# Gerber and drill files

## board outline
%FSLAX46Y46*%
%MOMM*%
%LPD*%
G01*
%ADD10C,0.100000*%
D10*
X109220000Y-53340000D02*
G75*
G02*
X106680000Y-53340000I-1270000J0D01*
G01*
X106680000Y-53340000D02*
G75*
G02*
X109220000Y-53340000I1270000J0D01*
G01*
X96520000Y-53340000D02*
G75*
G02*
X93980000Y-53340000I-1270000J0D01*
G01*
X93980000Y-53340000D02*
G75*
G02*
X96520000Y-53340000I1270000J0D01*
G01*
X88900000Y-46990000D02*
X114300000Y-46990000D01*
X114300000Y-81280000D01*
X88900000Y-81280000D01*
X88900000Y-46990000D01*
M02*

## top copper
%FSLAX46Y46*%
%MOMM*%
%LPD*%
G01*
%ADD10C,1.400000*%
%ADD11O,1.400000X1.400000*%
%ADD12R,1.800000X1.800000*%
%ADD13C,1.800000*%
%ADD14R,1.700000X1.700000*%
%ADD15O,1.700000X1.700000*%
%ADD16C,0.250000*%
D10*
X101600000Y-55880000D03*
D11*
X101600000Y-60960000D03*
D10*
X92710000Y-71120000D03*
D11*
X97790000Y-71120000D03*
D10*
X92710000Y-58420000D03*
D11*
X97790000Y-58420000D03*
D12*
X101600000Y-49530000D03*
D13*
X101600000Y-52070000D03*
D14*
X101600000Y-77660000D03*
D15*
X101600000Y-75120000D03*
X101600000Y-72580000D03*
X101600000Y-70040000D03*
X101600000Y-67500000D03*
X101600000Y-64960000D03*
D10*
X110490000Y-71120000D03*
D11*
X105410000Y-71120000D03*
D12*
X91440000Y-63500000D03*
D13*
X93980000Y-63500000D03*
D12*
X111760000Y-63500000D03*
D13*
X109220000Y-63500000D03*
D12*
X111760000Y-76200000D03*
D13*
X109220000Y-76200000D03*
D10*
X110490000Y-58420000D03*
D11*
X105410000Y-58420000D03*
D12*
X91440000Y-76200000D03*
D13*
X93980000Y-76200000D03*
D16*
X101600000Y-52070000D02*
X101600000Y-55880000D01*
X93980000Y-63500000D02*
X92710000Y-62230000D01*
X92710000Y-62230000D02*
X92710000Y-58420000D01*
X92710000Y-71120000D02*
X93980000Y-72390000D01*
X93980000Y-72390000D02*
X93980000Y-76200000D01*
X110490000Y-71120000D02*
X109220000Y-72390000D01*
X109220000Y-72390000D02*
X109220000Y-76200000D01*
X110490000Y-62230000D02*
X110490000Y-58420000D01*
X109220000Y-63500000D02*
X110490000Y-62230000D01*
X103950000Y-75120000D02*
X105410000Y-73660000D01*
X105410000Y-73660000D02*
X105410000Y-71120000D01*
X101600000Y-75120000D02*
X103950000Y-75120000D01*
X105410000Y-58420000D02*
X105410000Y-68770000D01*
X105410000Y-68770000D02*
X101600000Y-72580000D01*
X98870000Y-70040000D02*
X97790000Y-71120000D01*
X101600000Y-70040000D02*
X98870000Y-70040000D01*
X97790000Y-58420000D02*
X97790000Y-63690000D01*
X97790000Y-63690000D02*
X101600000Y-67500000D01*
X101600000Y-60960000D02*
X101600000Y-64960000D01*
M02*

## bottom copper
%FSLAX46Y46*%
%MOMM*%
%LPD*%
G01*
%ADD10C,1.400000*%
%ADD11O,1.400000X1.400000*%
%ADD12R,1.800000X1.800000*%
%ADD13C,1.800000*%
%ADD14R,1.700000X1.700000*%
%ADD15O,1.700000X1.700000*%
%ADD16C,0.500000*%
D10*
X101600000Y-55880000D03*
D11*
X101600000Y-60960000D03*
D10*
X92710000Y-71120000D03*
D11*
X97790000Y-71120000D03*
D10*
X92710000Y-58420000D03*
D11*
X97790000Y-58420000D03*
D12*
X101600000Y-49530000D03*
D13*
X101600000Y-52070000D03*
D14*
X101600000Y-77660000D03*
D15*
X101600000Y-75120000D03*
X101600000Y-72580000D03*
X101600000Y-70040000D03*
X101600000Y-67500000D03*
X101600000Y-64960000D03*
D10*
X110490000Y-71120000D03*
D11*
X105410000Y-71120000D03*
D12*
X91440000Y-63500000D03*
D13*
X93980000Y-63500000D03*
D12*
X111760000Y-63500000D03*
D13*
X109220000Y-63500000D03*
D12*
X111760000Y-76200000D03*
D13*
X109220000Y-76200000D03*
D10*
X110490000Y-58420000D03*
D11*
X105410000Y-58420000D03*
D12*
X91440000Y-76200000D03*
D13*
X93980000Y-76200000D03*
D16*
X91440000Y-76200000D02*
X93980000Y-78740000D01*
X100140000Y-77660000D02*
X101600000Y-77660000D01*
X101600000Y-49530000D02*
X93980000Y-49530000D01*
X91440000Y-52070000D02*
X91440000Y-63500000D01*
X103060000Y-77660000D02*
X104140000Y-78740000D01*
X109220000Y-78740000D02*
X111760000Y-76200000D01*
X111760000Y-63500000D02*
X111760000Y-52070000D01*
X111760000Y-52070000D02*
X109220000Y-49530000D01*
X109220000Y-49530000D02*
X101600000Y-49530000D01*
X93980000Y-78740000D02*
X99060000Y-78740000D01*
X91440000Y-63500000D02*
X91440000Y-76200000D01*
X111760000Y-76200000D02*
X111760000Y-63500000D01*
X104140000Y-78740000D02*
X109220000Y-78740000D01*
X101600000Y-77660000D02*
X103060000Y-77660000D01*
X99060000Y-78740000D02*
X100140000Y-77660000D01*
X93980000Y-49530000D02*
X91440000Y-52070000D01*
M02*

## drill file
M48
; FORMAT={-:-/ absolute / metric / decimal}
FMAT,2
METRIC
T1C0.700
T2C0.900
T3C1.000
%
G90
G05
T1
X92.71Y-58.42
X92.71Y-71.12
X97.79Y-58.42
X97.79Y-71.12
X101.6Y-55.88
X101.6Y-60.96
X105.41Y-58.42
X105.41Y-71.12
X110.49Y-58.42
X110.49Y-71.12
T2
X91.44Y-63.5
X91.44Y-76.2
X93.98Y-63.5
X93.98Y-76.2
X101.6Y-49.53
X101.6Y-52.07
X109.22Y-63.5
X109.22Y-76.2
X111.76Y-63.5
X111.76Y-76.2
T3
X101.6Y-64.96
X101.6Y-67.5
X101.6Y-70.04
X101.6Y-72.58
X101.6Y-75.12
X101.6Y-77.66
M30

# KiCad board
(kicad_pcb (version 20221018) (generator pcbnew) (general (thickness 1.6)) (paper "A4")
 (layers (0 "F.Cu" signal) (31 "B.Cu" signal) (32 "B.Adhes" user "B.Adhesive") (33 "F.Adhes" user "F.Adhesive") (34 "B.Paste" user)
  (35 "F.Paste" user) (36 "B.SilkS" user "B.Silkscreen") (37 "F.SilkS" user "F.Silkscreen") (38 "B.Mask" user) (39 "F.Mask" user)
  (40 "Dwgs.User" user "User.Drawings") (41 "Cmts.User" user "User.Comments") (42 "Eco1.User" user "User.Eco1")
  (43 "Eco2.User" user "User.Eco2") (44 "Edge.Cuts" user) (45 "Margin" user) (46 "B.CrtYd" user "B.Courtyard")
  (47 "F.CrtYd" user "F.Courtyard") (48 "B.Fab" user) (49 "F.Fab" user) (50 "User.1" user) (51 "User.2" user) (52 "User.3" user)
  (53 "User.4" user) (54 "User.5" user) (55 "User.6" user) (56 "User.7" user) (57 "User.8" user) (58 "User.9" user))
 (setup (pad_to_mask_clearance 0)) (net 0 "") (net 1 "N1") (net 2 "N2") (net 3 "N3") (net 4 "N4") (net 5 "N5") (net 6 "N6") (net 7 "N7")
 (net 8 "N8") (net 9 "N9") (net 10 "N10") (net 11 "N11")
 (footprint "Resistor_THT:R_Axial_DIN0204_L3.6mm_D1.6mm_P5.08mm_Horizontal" (layer "F.Cu") (at 101.6 55.88 -90)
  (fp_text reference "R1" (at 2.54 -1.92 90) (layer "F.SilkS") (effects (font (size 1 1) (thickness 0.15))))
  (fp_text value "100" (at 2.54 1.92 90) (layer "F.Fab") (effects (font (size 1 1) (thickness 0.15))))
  (pad "1" thru_hole circle (at 0 0 270) (size 1.4 1.4) (drill 0.7) (layers "*.Cu" "*.Mask") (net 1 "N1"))
  (pad "2" thru_hole oval (at 5.08 0 270) (size 1.4 1.4) (drill 0.7) (layers "*.Cu" "*.Mask") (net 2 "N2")))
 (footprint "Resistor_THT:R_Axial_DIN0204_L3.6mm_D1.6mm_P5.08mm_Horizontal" (layer "F.Cu") (at 92.71 71.12)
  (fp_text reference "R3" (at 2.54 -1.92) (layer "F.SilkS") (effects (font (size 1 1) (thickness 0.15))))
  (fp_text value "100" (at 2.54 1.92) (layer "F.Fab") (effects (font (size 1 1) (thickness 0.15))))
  (pad "1" thru_hole circle (at 0 0) (size 1.4 1.4) (drill 0.7) (layers "*.Cu" "*.Mask") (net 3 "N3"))
  (pad "2" thru_hole oval (at 5.08 0) (size 1.4 1.4) (drill 0.7) (layers "*.Cu" "*.Mask") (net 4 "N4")))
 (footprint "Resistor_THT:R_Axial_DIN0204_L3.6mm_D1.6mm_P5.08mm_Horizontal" (layer "F.Cu") (at 92.71 58.42)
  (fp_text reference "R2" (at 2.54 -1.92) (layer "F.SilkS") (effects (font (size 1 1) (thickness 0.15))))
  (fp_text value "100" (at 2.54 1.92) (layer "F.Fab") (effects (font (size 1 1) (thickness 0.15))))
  (pad "1" thru_hole circle (at 0 0) (size 1.4 1.4) (drill 0.7) (layers "*.Cu" "*.Mask") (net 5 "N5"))
  (pad "2" thru_hole oval (at 5.08 0) (size 1.4 1.4) (drill 0.7) (layers "*.Cu" "*.Mask") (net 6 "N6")))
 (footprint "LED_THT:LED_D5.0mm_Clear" (layer "F.Cu") (at 101.6 49.53 -90)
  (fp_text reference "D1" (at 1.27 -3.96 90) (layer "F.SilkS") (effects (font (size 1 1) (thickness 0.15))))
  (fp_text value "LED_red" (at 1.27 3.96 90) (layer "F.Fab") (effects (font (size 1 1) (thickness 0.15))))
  (pad "1" thru_hole rect (at 0 0 270) (size 1.8 1.8) (drill 0.9) (layers "*.Cu" "*.Mask") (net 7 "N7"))
  (pad "2" thru_hole circle (at 2.54 0 270) (size 1.8 1.8) (drill 0.9) (layers "*.Cu" "*.Mask") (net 1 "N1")))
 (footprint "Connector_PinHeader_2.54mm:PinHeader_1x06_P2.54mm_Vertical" (layer "F.Cu") (at 101.6 77.66 180)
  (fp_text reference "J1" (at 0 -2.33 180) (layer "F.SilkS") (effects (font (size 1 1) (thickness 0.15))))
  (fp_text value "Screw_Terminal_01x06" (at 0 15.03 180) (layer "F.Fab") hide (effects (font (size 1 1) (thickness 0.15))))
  (pad "1" thru_hole rect (at 0 0 180) (size 1.7 1.7) (drill 1) (layers "*.Cu" "*.Mask") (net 7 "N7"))
  (pad "2" thru_hole oval (at 0 2.54 180) (size 1.7 1.7) (drill 1) (layers "*.Cu" "*.Mask") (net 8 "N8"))
  (pad "3" thru_hole oval (at 0 5.08 180) (size 1.7 1.7) (drill 1) (layers "*.Cu" "*.Mask") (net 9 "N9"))
  (pad "4" thru_hole oval (at 0 7.62 180) (size 1.7 1.7) (drill 1) (layers "*.Cu" "*.Mask") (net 4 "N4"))
  (pad "5" thru_hole oval (at 0 10.16 180) (size 1.7 1.7) (drill 1) (layers "*.Cu" "*.Mask") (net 6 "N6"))
  (pad "6" thru_hole oval (at 0 12.7 180) (size 1.7 1.7) (drill 1) (layers "*.Cu" "*.Mask") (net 2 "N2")))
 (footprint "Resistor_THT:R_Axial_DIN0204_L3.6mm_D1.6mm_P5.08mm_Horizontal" (layer "F.Cu") (at 110.49 71.12 180)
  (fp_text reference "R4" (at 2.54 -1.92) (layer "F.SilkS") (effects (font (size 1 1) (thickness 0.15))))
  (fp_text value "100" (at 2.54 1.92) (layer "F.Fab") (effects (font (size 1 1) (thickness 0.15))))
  (pad "1" thru_hole circle (at 0 0 180) (size 1.4 1.4) (drill 0.7) (layers "*.Cu" "*.Mask") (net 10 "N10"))
  (pad "2" thru_hole oval (at 5.08 0 180) (size 1.4 1.4) (drill 0.7) (layers "*.Cu" "*.Mask") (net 8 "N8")))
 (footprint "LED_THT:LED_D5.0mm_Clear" (layer "F.Cu") (at 91.44 63.5)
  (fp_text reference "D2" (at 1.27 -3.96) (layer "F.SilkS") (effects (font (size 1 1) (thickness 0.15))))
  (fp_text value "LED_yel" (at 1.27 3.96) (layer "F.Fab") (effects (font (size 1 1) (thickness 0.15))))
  (pad "1" thru_hole rect (at 0 0) (size 1.8 1.8) (drill 0.9) (layers "*.Cu" "*.Mask") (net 7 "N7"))
  (pad "2" thru_hole circle (at 2.54 0) (size 1.8 1.8) (drill 0.9) (layers "*.Cu" "*.Mask") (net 5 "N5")))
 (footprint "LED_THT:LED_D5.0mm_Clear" (layer "F.Cu") (at 111.76 63.5 180)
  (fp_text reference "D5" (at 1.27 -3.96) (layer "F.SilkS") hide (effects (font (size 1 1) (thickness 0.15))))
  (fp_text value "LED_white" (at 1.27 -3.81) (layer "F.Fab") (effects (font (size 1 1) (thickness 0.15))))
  (pad "1" thru_hole rect (at 0 0 180) (size 1.8 1.8) (drill 0.9) (layers "*.Cu" "*.Mask") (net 7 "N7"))
  (pad "2" thru_hole circle (at 2.54 0 180) (size 1.8 1.8) (drill 0.9) (layers "*.Cu" "*.Mask") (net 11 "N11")))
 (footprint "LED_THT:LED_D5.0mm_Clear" (layer "F.Cu") (at 111.76 76.2 180)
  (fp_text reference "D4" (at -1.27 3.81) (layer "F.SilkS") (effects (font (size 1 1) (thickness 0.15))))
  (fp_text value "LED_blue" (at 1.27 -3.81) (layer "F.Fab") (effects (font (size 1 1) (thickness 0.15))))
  (pad "1" thru_hole rect (at 0 0 180) (size 1.8 1.8) (drill 0.9) (layers "*.Cu" "*.Mask") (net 7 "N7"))
  (pad "2" thru_hole circle (at 2.54 0 180) (size 1.8 1.8) (drill 0.9) (layers "*.Cu" "*.Mask") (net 10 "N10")))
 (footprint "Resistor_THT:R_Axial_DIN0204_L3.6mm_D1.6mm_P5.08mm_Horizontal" (layer "F.Cu") (at 110.49 58.42 180)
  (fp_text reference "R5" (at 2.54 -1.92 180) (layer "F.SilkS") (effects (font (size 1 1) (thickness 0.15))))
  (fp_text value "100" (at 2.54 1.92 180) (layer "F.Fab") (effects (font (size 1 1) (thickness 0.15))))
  (pad "1" thru_hole circle (at 0 0 180) (size 1.4 1.4) (drill 0.7) (layers "*.Cu" "*.Mask") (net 11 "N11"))
  (pad "2" thru_hole oval (at 5.08 0 180) (size 1.4 1.4) (drill 0.7) (layers "*.Cu" "*.Mask") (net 9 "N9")))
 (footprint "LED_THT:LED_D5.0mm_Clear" (layer "F.Cu") (at 91.44 76.2)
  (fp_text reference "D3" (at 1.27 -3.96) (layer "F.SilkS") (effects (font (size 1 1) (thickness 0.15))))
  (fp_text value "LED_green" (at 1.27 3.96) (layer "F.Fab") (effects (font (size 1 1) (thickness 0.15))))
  (pad "1" thru_hole rect (at 0 0) (size 1.8 1.8) (drill 0.9) (layers "*.Cu" "*.Mask") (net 7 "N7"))
  (pad "2" thru_hole circle (at 2.54 0) (size 1.8 1.8) (drill 0.9) (layers "*.Cu" "*.Mask") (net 3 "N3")))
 (gr_circle (center 107.95 53.34) (end 109.22 53.34) (stroke (width 0.1) (type default)) (fill none) (layer "Edge.Cuts"))
 (gr_circle (center 95.25 53.34) (end 93.98 53.34) (stroke (width 0.1) (type default)) (fill none) (layer "Edge.Cuts"))
 (gr_rect (start 88.9 46.99) (end 114.3 81.28) (stroke (width 0.1) (type default)) (fill none) (layer "Edge.Cuts"))
 (segment (start 101.6 52.07) (end 101.6 55.88) (width 0.25) (layer "F.Cu") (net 1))
 (segment (start 93.98 63.5) (end 92.71 62.23) (width 0.25) (layer "F.Cu") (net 5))
 (segment (start 92.71 62.23) (end 92.71 58.42) (width 0.25) (layer "F.Cu") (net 5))
 (segment (start 92.71 71.12) (end 93.98 72.39) (width 0.25) (layer "F.Cu") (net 3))
 (segment (start 93.98 72.39) (end 93.98 76.2) (width 0.25) (layer "F.Cu") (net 3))
 (segment (start 110.49 71.12) (end 109.22 72.39) (width 0.25) (layer "F.Cu") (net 10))
 (segment (start 109.22 72.39) (end 109.22 76.2) (width 0.25) (layer "F.Cu") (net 10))
 (segment (start 110.49 62.23) (end 110.49 58.42) (width 0.25) (layer "F.Cu") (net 11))
 (segment (start 109.22 63.5) (end 110.49 62.23) (width 0.25) (layer "F.Cu") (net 11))
 (segment (start 91.44 76.2) (end 93.98 78.74) (width 0.5) (layer "B.Cu") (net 7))
 (segment (start 100.14 77.66) (end 101.6 77.66) (width 0.5) (layer "B.Cu") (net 7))
 (segment (start 101.6 49.53) (end 93.98 49.53) (width 0.5) (layer "B.Cu") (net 7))
 (segment (start 91.44 52.07) (end 91.44 63.5) (width 0.5) (layer "B.Cu") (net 7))
 (segment (start 103.06 77.66) (end 104.14 78.74) (width 0.5) (layer "B.Cu") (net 7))
 (segment (start 109.22 78.74) (end 111.76 76.2) (width 0.5) (layer "B.Cu") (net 7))
 (segment (start 111.76 63.5) (end 111.76 52.07) (width 0.5) (layer "B.Cu") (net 7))
 (segment (start 111.76 52.07) (end 109.22 49.53) (width 0.5) (layer "B.Cu") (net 7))
 (segment (start 109.22 49.53) (end 101.6 49.53) (width 0.5) (layer "B.Cu") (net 7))
 (segment (start 93.98 78.74) (end 99.06 78.74) (width 0.5) (layer "B.Cu") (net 7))
 (segment (start 91.44 63.5) (end 91.44 76.2) (width 0.5) (layer "B.Cu") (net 7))
 (segment (start 111.76 76.2) (end 111.76 63.5) (width 0.5) (layer "B.Cu") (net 7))
 (segment (start 104.14 78.74) (end 109.22 78.74) (width 0.5) (layer "B.Cu") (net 7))
 (segment (start 101.6 77.66) (end 103.06 77.66) (width 0.5) (layer "B.Cu") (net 7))
 (segment (start 99.06 78.74) (end 100.14 77.66) (width 0.5) (layer "B.Cu") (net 7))
 (segment (start 93.98 49.53) (end 91.44 52.07) (width 0.5) (layer "B.Cu") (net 7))
 (segment (start 103.95 75.12) (end 105.41 73.66) (width 0.25) (layer "F.Cu") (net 8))
 (segment (start 105.41 73.66) (end 105.41 71.12) (width 0.25) (layer "F.Cu") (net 8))
 (segment (start 101.6 75.12) (end 103.95 75.12) (width 0.25) (layer "F.Cu") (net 8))
 (segment (start 105.41 58.42) (end 105.41 68.77) (width 0.25) (layer "F.Cu") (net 9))
 (segment (start 105.41 68.77) (end 101.6 72.58) (width 0.25) (layer "F.Cu") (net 9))
 (segment (start 98.87 70.04) (end 97.79 71.12) (width 0.25) (layer "F.Cu") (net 4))
 (segment (start 101.6 70.04) (end 98.87 70.04) (width 0.25) (layer "F.Cu") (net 4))
 (segment (start 97.79 58.42) (end 97.79 63.69) (width 0.25) (layer "F.Cu") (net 6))
 (segment (start 97.79 63.69) (end 101.6 67.5) (width 0.25) (layer "F.Cu") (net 6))
 (segment (start 101.6 60.96) (end 101.6 64.96) (width 0.25) (layer "F.Cu") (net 2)))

